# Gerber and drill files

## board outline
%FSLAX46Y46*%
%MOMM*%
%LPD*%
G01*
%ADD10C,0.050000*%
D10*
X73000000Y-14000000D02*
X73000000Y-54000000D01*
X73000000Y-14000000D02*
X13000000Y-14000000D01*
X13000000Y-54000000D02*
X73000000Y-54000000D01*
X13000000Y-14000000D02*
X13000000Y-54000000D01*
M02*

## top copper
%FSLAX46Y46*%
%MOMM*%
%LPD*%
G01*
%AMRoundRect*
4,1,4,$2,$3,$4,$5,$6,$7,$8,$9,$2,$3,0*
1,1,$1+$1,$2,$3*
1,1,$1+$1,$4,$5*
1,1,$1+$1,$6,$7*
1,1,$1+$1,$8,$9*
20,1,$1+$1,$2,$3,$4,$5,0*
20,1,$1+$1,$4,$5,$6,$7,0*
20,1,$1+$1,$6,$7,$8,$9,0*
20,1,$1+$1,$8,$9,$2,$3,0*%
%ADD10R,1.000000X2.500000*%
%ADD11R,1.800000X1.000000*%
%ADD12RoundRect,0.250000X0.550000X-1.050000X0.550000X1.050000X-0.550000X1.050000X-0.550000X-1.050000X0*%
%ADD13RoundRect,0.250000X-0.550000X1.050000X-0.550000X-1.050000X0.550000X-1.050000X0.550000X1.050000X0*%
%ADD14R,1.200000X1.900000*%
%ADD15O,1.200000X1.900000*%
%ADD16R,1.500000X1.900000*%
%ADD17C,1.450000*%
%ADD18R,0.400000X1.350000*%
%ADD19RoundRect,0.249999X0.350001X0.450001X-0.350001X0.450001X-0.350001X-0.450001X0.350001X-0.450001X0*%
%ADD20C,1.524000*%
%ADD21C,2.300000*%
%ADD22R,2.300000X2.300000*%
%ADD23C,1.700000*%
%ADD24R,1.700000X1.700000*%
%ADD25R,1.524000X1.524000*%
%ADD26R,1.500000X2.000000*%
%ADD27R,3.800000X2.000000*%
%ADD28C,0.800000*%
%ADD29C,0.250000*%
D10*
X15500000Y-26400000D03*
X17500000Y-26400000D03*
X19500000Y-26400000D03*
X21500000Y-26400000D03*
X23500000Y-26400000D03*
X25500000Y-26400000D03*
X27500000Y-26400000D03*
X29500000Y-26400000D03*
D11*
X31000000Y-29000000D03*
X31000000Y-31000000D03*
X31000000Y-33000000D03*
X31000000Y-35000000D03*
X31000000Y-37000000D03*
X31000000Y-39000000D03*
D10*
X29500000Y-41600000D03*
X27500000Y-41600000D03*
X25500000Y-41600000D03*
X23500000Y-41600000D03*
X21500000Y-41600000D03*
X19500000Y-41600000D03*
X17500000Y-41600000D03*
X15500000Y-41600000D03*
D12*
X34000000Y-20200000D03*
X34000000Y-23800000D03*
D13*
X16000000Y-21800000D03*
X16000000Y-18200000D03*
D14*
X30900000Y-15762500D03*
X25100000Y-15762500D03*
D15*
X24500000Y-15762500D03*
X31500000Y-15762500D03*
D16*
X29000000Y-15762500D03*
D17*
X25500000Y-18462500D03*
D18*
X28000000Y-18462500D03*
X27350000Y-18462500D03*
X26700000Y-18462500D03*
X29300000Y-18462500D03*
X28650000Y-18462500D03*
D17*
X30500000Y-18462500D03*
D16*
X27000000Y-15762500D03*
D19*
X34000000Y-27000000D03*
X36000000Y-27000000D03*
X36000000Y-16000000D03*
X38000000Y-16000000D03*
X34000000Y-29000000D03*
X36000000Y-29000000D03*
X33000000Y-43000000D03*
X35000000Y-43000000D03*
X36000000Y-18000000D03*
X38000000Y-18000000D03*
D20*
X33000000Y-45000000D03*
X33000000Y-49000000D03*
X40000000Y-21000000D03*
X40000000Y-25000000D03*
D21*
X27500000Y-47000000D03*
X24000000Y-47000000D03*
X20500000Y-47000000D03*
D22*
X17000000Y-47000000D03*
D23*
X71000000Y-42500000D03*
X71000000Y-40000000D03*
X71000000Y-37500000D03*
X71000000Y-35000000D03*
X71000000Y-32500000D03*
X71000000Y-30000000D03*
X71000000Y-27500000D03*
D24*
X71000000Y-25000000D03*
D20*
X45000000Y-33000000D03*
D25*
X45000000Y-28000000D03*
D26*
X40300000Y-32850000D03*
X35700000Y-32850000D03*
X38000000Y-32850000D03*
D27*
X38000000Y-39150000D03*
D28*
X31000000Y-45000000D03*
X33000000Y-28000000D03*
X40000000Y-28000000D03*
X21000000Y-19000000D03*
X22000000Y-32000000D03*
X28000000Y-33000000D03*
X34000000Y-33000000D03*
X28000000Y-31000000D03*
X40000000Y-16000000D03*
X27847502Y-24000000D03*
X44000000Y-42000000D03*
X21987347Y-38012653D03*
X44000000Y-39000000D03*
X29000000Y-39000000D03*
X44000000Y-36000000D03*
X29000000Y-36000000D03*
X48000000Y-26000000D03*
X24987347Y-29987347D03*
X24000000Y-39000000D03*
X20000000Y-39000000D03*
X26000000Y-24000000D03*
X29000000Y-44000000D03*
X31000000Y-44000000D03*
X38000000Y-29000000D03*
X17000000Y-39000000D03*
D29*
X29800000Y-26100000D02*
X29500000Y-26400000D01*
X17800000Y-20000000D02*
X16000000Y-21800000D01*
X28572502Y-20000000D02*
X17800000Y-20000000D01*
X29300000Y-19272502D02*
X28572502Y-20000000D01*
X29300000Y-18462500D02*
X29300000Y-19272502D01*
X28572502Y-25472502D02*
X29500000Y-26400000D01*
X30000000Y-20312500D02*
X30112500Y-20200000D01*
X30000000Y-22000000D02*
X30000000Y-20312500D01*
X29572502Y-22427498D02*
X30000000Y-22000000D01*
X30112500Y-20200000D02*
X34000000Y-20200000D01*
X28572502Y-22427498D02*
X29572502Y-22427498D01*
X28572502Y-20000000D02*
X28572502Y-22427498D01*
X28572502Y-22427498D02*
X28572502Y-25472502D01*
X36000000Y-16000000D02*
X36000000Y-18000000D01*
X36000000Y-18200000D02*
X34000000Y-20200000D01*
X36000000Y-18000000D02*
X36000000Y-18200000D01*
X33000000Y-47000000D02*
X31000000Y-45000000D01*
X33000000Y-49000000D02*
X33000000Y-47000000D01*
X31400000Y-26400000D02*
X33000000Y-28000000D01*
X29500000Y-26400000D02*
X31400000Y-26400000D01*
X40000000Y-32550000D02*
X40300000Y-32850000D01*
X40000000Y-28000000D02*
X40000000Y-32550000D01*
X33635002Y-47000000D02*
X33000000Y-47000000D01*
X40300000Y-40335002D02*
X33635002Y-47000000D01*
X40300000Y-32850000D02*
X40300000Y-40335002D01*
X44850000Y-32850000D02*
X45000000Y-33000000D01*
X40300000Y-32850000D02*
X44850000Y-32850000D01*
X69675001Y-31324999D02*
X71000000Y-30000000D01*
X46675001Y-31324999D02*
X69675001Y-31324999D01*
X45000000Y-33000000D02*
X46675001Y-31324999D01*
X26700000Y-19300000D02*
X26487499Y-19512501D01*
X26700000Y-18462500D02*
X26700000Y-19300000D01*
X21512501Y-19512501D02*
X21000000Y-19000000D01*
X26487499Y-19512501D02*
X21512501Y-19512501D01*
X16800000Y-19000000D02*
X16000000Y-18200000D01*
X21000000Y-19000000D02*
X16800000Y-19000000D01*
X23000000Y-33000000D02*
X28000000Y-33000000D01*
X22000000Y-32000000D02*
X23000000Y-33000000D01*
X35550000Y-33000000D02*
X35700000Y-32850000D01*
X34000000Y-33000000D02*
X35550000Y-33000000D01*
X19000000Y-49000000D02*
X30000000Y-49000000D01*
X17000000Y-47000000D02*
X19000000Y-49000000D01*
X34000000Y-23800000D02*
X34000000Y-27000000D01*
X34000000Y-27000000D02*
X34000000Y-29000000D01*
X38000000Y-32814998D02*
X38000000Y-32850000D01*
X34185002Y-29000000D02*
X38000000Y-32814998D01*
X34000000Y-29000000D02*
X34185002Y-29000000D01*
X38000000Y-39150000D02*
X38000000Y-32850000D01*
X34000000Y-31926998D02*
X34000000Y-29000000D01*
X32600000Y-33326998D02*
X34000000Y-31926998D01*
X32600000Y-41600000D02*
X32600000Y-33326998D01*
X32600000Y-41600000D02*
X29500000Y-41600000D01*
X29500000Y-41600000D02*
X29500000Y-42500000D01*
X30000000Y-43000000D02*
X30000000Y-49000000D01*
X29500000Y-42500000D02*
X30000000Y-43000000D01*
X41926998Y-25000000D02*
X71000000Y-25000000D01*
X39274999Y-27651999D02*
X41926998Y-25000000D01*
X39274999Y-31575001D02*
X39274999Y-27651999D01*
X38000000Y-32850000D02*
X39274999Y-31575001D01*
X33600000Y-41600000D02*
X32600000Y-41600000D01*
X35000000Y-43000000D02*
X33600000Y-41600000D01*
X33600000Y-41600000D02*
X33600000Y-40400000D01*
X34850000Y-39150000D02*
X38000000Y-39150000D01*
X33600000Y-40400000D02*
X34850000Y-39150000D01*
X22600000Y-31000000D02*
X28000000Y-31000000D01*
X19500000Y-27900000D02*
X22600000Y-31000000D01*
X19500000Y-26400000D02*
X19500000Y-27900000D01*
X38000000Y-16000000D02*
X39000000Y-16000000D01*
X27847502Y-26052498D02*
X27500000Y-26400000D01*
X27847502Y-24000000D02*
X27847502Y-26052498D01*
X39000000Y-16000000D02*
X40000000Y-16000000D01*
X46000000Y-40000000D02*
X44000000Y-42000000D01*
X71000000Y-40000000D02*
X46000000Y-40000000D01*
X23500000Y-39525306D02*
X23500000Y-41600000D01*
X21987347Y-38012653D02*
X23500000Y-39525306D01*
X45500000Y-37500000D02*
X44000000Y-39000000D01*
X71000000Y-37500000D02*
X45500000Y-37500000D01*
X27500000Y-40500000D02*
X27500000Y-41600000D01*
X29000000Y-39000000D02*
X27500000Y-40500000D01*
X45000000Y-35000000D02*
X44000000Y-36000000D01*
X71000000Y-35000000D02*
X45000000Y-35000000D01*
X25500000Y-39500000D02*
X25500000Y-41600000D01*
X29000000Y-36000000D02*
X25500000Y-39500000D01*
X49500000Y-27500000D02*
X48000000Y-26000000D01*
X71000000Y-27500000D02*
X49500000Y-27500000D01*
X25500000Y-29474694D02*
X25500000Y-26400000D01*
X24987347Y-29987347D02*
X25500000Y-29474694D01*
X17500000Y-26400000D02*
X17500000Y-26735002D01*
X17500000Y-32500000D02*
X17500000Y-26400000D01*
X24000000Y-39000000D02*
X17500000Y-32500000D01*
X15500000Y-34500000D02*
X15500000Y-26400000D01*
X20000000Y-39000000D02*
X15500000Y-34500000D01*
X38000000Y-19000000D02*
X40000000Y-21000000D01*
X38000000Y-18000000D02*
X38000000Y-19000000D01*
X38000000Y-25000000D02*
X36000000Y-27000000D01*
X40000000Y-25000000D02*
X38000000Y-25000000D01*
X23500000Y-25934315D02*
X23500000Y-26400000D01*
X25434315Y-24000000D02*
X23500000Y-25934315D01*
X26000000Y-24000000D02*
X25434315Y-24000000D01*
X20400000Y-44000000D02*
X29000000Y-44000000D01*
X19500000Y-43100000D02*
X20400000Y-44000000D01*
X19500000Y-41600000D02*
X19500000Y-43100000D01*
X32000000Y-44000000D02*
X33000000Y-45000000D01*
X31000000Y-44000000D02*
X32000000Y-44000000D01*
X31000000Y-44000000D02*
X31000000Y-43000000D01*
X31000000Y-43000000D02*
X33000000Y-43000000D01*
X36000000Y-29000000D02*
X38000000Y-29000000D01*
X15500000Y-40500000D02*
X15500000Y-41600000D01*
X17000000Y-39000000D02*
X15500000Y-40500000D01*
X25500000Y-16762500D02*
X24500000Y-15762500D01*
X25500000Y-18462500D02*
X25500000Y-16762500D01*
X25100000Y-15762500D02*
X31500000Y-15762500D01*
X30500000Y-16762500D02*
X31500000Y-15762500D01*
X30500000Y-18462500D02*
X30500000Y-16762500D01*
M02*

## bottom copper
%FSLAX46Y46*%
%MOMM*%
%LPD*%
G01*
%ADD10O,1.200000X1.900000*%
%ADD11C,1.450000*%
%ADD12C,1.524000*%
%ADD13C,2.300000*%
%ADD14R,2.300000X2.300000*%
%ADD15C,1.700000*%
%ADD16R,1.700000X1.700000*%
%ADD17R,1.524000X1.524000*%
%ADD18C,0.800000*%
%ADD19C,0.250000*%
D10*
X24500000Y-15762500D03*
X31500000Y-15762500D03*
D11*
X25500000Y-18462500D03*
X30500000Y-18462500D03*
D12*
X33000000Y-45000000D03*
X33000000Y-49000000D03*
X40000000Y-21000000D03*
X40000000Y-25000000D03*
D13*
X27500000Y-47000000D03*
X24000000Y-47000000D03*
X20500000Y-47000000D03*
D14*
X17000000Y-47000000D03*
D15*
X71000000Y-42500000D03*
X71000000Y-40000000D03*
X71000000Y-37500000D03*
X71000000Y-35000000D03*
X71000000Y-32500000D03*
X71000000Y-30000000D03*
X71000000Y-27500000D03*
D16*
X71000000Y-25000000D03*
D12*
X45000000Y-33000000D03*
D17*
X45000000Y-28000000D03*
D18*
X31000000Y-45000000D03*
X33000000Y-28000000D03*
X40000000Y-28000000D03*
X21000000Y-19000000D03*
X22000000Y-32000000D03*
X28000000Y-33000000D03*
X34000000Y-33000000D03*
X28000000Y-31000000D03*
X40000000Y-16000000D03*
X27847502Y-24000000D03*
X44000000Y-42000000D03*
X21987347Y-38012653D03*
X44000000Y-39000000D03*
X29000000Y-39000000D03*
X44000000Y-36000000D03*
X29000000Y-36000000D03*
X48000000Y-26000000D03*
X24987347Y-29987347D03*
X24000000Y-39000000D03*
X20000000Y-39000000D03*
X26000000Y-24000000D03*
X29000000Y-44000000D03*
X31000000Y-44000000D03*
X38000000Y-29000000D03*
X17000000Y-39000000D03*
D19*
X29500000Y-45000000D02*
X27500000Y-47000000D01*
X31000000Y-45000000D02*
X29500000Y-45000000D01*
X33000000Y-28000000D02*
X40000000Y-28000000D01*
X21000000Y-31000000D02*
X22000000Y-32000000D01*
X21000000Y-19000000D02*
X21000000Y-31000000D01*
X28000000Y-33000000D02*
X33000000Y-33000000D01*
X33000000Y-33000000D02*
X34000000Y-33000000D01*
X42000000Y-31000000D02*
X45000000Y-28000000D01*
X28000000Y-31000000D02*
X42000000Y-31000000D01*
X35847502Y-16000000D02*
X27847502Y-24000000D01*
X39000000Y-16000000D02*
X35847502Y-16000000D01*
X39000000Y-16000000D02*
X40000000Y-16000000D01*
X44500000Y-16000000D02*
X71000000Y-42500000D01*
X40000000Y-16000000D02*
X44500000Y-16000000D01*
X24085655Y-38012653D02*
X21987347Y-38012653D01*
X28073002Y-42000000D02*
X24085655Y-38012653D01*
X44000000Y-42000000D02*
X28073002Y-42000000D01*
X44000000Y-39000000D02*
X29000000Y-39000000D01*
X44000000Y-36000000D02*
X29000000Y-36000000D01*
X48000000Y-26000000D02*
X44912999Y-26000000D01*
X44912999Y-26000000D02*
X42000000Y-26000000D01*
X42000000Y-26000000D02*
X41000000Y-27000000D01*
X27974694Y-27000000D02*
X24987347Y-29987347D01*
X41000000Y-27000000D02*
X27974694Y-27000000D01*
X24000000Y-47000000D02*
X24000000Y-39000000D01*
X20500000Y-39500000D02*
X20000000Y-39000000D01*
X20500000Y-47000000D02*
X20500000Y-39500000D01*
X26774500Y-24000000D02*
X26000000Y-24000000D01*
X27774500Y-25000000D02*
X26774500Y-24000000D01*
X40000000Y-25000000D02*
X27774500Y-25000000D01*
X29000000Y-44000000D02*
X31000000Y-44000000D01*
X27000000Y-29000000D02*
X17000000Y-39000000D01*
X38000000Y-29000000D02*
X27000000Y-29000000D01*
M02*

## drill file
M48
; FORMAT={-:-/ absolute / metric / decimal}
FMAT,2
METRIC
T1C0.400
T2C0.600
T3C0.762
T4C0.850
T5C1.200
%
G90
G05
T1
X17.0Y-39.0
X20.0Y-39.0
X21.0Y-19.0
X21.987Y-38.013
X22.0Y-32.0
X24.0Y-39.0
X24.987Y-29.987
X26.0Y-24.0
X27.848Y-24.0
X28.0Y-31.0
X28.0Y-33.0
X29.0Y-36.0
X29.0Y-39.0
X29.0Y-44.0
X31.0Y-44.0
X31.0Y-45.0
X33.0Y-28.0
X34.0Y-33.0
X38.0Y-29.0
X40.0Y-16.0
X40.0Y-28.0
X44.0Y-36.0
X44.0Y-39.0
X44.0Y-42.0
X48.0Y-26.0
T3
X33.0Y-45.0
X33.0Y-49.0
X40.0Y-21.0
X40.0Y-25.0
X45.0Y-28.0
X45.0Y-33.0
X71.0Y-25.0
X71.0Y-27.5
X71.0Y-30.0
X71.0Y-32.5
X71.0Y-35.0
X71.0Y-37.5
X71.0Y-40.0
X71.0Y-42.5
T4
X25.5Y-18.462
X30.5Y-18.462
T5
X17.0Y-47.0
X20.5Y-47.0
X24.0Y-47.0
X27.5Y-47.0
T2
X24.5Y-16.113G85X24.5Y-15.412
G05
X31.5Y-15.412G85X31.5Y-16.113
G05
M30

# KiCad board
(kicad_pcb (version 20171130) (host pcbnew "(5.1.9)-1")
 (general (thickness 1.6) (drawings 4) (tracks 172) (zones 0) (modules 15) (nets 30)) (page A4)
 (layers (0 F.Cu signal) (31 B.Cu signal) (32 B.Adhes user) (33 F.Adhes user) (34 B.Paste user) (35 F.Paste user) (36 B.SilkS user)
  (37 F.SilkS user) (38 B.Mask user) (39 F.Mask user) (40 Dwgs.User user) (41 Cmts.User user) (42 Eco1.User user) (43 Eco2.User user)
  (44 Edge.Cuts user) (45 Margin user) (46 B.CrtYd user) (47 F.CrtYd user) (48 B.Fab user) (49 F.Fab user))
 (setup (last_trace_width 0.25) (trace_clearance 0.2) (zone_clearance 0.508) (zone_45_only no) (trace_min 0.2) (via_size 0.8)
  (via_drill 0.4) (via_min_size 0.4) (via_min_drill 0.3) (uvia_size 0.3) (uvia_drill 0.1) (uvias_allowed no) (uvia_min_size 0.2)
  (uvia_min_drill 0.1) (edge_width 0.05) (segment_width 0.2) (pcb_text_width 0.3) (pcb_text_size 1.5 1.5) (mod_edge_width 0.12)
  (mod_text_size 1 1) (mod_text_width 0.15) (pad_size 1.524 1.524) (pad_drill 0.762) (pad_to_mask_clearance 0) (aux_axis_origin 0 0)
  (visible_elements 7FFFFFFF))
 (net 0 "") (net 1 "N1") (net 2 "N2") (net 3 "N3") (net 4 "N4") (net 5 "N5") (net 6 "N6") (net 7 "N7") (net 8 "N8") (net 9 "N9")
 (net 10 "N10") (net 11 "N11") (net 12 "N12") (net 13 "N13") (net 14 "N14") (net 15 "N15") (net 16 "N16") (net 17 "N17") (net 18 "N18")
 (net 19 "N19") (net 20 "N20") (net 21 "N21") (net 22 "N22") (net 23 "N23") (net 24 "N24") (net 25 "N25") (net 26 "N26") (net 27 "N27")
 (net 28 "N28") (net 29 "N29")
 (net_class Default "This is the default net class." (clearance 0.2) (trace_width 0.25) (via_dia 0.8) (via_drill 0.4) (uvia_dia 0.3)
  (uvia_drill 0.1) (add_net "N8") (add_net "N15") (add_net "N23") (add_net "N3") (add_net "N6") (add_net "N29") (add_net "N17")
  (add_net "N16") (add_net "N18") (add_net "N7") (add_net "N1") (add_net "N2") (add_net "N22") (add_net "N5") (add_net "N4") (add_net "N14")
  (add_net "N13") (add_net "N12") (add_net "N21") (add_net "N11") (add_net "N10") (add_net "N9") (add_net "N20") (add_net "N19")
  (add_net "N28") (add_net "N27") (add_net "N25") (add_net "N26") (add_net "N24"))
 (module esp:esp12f (layer F.Cu) (at 19 34 90)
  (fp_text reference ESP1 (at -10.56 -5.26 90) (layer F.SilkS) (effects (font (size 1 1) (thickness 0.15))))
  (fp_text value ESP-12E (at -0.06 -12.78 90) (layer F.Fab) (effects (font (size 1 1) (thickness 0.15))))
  (pad 16 smd rect (at 7.6 -3.5 90) (size 2.5 1) (layers F.Cu F.Paste F.Mask) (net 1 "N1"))
  (pad 15 smd rect (at 7.6 -1.5 90) (size 2.5 1) (layers F.Cu F.Paste F.Mask) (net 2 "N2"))
  (pad 14 smd rect (at 7.6 0.5 90) (size 2.5 1) (layers F.Cu F.Paste F.Mask) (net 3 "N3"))
  (pad 13 smd rect (at 7.6 2.5 90) (size 2.5 1) (layers F.Cu F.Paste F.Mask) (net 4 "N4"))
  (pad 12 smd rect (at 7.6 4.5 90) (size 2.5 1) (layers F.Cu F.Paste F.Mask) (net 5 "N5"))
  (pad 11 smd rect (at 7.6 6.5 90) (size 2.5 1) (layers F.Cu F.Paste F.Mask) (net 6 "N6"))
  (pad 10 smd rect (at 7.6 8.5 90) (size 2.5 1) (layers F.Cu F.Paste F.Mask) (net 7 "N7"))
  (pad 9 smd rect (at 7.6 10.5 90) (size 2.5 1) (layers F.Cu F.Paste F.Mask) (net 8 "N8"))
  (pad 22 smd rect (at 5 12 90) (size 1 1.8) (layers F.Cu F.Paste F.Mask) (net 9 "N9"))
  (pad 21 smd rect (at 3 12 90) (size 1 1.8) (layers F.Cu F.Paste F.Mask) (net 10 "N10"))
  (pad 20 smd rect (at 1 12 90) (size 1 1.8) (layers F.Cu F.Paste F.Mask) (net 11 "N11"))
  (pad 19 smd rect (at -1 12 90) (size 1 1.8) (layers F.Cu F.Paste F.Mask) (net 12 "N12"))
  (pad 18 smd rect (at -3 12 90) (size 1 1.8) (layers F.Cu F.Paste F.Mask) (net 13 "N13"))
  (pad 17 smd rect (at -5 12 90) (size 1 1.8) (layers F.Cu F.Paste F.Mask) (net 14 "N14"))
  (pad 8 smd rect (at -7.6 10.5 90) (size 2.5 1) (layers F.Cu F.Paste F.Mask) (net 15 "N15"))
  (pad 7 smd rect (at -7.6 8.5 90) (size 2.5 1) (layers F.Cu F.Paste F.Mask) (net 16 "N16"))
  (pad 6 smd rect (at -7.6 6.5 90) (size 2.5 1) (layers F.Cu F.Paste F.Mask) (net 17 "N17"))
  (pad 5 smd rect (at -7.6 4.5 90) (size 2.5 1) (layers F.Cu F.Paste F.Mask) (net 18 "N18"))
  (pad 4 smd rect (at -7.6 2.5 90) (size 2.5 1) (layers F.Cu F.Paste F.Mask) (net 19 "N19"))
  (pad 3 smd rect (at -7.6 0.5 90) (size 2.5 1) (layers F.Cu F.Paste F.Mask) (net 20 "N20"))
  (pad 2 smd rect (at -7.6 -1.5 90) (size 2.5 1) (layers F.Cu F.Paste F.Mask) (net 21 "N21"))
  (pad 1 smd rect (at -7.6 -3.5 90) (size 2.5 1) (layers F.Cu F.Paste F.Mask) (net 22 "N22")))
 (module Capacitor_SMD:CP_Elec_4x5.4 (layer F.Cu) (at 34 22 90)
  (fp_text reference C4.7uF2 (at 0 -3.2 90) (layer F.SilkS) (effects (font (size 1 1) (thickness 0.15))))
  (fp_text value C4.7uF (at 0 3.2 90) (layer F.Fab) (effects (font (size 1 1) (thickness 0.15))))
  (pad 2 smd roundrect (at 1.8 0 90) (size 2.6 1.6) (layers F.Cu F.Paste F.Mask) (roundrect_rratio 0.15625) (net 8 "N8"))
  (pad 1 smd roundrect (at -1.8 0 90) (size 2.6 1.6) (layers F.Cu F.Paste F.Mask) (roundrect_rratio 0.15625) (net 15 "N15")))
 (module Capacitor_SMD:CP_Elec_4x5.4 (layer F.Cu) (at 16 20 270)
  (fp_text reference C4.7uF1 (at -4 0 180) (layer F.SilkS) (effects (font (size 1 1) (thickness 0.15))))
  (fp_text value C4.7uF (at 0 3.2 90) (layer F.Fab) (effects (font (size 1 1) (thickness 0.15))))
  (pad 2 smd roundrect (at 1.8 0 270) (size 2.6 1.6) (layers F.Cu F.Paste F.Mask) (roundrect_rratio 0.15625) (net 8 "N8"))
  (pad 1 smd roundrect (at -1.8 0 270) (size 2.6 1.6) (layers F.Cu F.Paste F.Mask) (roundrect_rratio 0.15625) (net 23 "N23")))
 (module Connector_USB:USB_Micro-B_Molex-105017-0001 (layer F.Cu) (at 28 17 180)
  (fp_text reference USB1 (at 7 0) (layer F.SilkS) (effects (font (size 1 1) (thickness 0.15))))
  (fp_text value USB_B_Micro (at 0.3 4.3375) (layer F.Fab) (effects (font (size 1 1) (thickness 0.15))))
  (pad 6 smd rect (at -2.9 1.2375 180) (size 1.2 1.9) (layers F.Cu F.Mask) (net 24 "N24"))
  (pad 6 smd rect (at 2.9 1.2375 180) (size 1.2 1.9) (layers F.Cu F.Mask) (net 24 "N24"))
  (pad 6 thru_hole oval (at 3.5 1.2375 180) (size 1.2 1.9) (drill oval 0.6 1.3) (layers *.Cu *.Mask) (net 24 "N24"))
  (pad 6 thru_hole oval (at -3.5 1.2375) (size 1.2 1.9) (drill oval 0.6 1.3) (layers *.Cu *.Mask) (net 24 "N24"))
  (pad 6 smd rect (at -1 1.2375 180) (size 1.5 1.9) (layers F.Cu F.Paste F.Mask) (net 24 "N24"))
  (pad 6 thru_hole circle (at 2.5 -1.4625 180) (size 1.45 1.45) (drill 0.85) (layers *.Cu *.Mask) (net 24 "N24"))
  (pad 3 smd rect (at 0 -1.4625 180) (size 0.4 1.35) (layers F.Cu F.Paste F.Mask) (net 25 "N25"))
  (pad 4 smd rect (at 0.65 -1.4625 180) (size 0.4 1.35) (layers F.Cu F.Paste F.Mask) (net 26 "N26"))
  (pad 5 smd rect (at 1.3 -1.4625 180) (size 0.4 1.35) (layers F.Cu F.Paste F.Mask) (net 23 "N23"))
  (pad 1 smd rect (at -1.3 -1.4625 180) (size 0.4 1.35) (layers F.Cu F.Paste F.Mask) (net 8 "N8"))
  (pad 2 smd rect (at -0.65 -1.4625 180) (size 0.4 1.35) (layers F.Cu F.Paste F.Mask) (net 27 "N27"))
  (pad 6 thru_hole circle (at -2.5 -1.4625 180) (size 1.45 1.45) (drill 0.85) (layers *.Cu *.Mask) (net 24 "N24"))
  (pad 6 smd rect (at 1 1.2375 180) (size 1.5 1.9) (layers F.Cu F.Paste F.Mask) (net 24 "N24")))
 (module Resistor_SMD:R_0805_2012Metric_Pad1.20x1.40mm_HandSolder (layer F.Cu) (at 35 27 180)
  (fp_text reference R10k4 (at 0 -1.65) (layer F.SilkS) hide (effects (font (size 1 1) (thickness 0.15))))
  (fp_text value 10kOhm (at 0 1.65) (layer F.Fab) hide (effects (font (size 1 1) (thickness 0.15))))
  (pad 2 smd roundrect (at 1 0 180) (size 1.2 1.4) (layers F.Cu F.Paste F.Mask) (roundrect_rratio 0.2083325) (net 15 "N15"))
  (pad 1 smd roundrect (at -1 0 180) (size 1.2 1.4) (layers F.Cu F.Paste F.Mask) (roundrect_rratio 0.2083325) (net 5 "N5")))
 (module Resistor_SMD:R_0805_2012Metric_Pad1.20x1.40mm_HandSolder (layer F.Cu) (at 37 16 180)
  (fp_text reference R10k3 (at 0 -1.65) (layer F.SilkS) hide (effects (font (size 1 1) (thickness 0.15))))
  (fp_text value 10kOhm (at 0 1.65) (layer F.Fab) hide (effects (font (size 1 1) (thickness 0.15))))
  (pad 2 smd roundrect (at 1 0 180) (size 1.2 1.4) (layers F.Cu F.Paste F.Mask) (roundrect_rratio 0.2083325) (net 8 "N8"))
  (pad 1 smd roundrect (at -1 0 180) (size 1.2 1.4) (layers F.Cu F.Paste F.Mask) (roundrect_rratio 0.2083325) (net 7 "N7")))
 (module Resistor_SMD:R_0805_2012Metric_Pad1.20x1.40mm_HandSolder (layer F.Cu) (at 35 29 180)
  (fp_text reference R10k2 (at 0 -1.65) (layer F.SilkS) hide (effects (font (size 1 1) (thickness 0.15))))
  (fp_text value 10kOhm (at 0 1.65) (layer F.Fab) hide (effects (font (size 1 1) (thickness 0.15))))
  (pad 2 smd roundrect (at 1 0 180) (size 1.2 1.4) (layers F.Cu F.Paste F.Mask) (roundrect_rratio 0.2083325) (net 15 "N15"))
  (pad 1 smd roundrect (at -1 0 180) (size 1.2 1.4) (layers F.Cu F.Paste F.Mask) (roundrect_rratio 0.2083325) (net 22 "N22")))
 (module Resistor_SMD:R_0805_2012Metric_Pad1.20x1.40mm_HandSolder (layer F.Cu) (at 34 43 180)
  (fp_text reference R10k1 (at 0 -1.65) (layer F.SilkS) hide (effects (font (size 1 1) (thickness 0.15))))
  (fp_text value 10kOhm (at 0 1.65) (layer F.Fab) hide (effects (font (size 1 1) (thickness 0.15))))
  (pad 2 smd roundrect (at 1 0 180) (size 1.2 1.4) (layers F.Cu F.Paste F.Mask) (roundrect_rratio 0.2083325) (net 20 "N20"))
  (pad 1 smd roundrect (at -1 0 180) (size 1.2 1.4) (layers F.Cu F.Paste F.Mask) (roundrect_rratio 0.2083325) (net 15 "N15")))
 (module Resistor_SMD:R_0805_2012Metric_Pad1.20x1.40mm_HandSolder (layer F.Cu) (at 37 18 180)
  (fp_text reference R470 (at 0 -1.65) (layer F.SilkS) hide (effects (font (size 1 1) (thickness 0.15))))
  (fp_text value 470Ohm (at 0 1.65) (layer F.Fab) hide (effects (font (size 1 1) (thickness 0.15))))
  (pad 2 smd roundrect (at 1 0 180) (size 1.2 1.4) (layers F.Cu F.Paste F.Mask) (roundrect_rratio 0.2083325) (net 8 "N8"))
  (pad 1 smd roundrect (at -1 0 180) (size 1.2 1.4) (layers F.Cu F.Paste F.Mask) (roundrect_rratio 0.2083325) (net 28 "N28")))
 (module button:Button (layer F.Cu) (at 33 47 180)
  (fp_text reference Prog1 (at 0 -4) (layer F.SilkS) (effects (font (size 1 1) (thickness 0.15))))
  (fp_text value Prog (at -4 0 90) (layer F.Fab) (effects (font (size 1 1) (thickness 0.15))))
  (pad 2 thru_hole circle (at 0 2 180) (size 1.524 1.524) (drill 0.762) (layers *.Cu *.Mask) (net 20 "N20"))
  (pad 1 thru_hole circle (at 0 -2 180) (size 1.524 1.524) (drill 0.762) (layers *.Cu *.Mask) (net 8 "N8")))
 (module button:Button (layer F.Cu) (at 40 23 180)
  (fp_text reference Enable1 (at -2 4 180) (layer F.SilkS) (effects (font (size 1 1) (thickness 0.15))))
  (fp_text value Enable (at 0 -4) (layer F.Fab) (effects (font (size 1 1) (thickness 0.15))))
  (pad 2 thru_hole circle (at 0 2 180) (size 1.524 1.524) (drill 0.762) (layers *.Cu *.Mask) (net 28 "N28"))
  (pad 1 thru_hole circle (at 0 -2 180) (size 1.524 1.524) (drill 0.762) (layers *.Cu *.Mask) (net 5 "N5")))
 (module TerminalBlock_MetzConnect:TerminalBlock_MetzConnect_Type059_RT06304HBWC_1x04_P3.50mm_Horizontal (layer F.Cu) (at 17 47)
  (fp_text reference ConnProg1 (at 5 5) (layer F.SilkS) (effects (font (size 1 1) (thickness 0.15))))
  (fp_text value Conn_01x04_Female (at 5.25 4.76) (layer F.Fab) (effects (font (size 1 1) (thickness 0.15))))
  (pad 4 thru_hole circle (at 10.5 0) (size 2.3 2.3) (drill 1.2) (layers *.Cu *.Mask) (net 8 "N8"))
  (pad 3 thru_hole circle (at 7 0) (size 2.3 2.3) (drill 1.2) (layers *.Cu *.Mask) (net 2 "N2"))
  (pad 2 thru_hole circle (at 3.5 0) (size 2.3 2.3) (drill 1.2) (layers *.Cu *.Mask) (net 1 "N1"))
  (pad 1 thru_hole rect (at 0 0) (size 2.3 2.3) (drill 1.2) (layers *.Cu *.Mask) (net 15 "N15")))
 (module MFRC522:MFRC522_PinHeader (layer F.Cu) (at 73 24 270)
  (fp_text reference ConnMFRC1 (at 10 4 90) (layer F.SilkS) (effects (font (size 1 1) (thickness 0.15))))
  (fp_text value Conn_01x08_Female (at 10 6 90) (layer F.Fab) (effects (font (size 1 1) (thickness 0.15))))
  (pad 8 thru_hole circle (at 18.5 2 270) (size 1.7 1.7) (drill 0.762) (layers *.Cu *.Mask) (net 7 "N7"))
  (pad 7 thru_hole circle (at 16 2 270) (size 1.7 1.7) (drill 0.762) (layers *.Cu *.Mask) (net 18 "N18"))
  (pad 6 thru_hole circle (at 13.5 2 270) (size 1.7 1.7) (drill 0.762) (layers *.Cu *.Mask) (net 16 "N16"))
  (pad 5 thru_hole circle (at 11 2 270) (size 1.7 1.7) (drill 0.762) (layers *.Cu *.Mask) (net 17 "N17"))
  (pad 4 thru_hole circle (at 8.5 2 270) (size 1.7 1.7) (drill 0.762) (layers *.Cu *.Mask) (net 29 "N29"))
  (pad 3 thru_hole circle (at 6 2 270) (size 1.7 1.7) (drill 0.762) (layers *.Cu *.Mask) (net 8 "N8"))
  (pad 2 thru_hole circle (at 3.5 2 270) (size 1.7 1.7) (drill 0.762) (layers *.Cu *.Mask) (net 6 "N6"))
  (pad 1 thru_hole rect (at 1 2 270) (size 1.7 1.7) (drill 0.762) (layers *.Cu *.Mask) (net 15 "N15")))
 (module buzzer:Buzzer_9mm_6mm (layer F.Cu) (at 46 27 270)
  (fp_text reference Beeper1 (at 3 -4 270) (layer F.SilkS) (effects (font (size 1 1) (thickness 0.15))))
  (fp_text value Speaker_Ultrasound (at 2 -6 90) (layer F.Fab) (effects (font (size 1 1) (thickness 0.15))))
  (pad 2 thru_hole circle (at 6 1 270) (size 1.524 1.524) (drill 0.762) (layers *.Cu *.Mask) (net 8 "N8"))
  (pad 1 thru_hole rect (at 1 1 270) (size 1.524 1.524) (drill 0.762) (layers *.Cu *.Mask) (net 3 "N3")))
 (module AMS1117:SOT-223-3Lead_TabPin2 (layer F.Cu) (at 38 36 270)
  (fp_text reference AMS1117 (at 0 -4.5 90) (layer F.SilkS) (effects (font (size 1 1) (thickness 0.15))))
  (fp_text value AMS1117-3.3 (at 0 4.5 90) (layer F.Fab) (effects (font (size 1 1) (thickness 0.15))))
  (pad 1 smd rect (at -3.15 -2.3 270) (size 2 1.5) (layers F.Cu F.Paste F.Mask) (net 8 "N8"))
  (pad 3 smd rect (at -3.15 2.3 270) (size 2 1.5) (layers F.Cu F.Paste F.Mask) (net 23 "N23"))
  (pad 2 smd rect (at -3.15 0 270) (size 2 1.5) (layers F.Cu F.Paste F.Mask) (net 15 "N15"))
  (pad 2 smd rect (at 3.15 0 270) (size 2 3.8) (layers F.Cu F.Paste F.Mask) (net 15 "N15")))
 (gr_line (start 73 14) (end 73 54) (layer Edge.Cuts) (width 0.05))
 (gr_line (start 73 14) (end 13 14) (layer Edge.Cuts) (width 0.05))
 (gr_line (start 13 54) (end 73 54) (layer Edge.Cuts) (width 0.05))
 (gr_line (start 13 14) (end 13 54) (layer Edge.Cuts) (width 0.05))
 (segment (start 29.8 26.1) (end 29.5 26.4) (width 0.25) (layer F.Cu) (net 8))
 (segment (start 17.8 20) (end 16 21.8) (width 0.25) (layer F.Cu) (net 8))
 (segment (start 28.572502 20) (end 17.8 20) (width 0.25) (layer F.Cu) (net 8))
 (segment (start 29.3 19.272502) (end 28.572502 20) (width 0.25) (layer F.Cu) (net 8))
 (segment (start 29.3 18.4625) (end 29.3 19.272502) (width 0.25) (layer F.Cu) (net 8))
 (segment (start 28.572502 25.472502) (end 29.5 26.4) (width 0.25) (layer F.Cu) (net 8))
 (segment (start 30 20.3125) (end 30.1125 20.2) (width 0.25) (layer F.Cu) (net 8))
 (segment (start 30 22) (end 30 20.3125) (width 0.25) (layer F.Cu) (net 8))
 (segment (start 29.572502 22.427498) (end 30 22) (width 0.25) (layer F.Cu) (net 8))
 (segment (start 30.1125 20.2) (end 34 20.2) (width 0.25) (layer F.Cu) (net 8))
 (segment (start 28.572502 22.427498) (end 29.572502 22.427498) (width 0.25) (layer F.Cu) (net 8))
 (segment (start 28.572502 20) (end 28.572502 22.427498) (width 0.25) (layer F.Cu) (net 8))
 (segment (start 28.572502 22.427498) (end 28.572502 25.472502) (width 0.25) (layer F.Cu) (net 8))
 (segment (start 36 16) (end 36 18) (width 0.25) (layer F.Cu) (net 8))
 (segment (start 36 18.2) (end 34 20.2) (width 0.25) (layer F.Cu) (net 8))
 (segment (start 36 18) (end 36 18.2) (width 0.25) (layer F.Cu) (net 8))
 (via (at 31 45) (size 0.8) (drill 0.4) (layers F.Cu B.Cu) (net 8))
 (segment (start 33 47) (end 31 45) (width 0.25) (layer F.Cu) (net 8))
 (segment (start 33 49) (end 33 47) (width 0.25) (layer F.Cu) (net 8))
 (segment (start 29.5 45) (end 27.5 47) (width 0.25) (layer B.Cu) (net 8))
 (segment (start 31 45) (end 29.5 45) (width 0.25) (layer B.Cu) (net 8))
 (via (at 33 28) (size 0.8) (drill 0.4) (layers F.Cu B.Cu) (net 8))
 (segment (start 31.4 26.4) (end 33 28) (width 0.25) (layer F.Cu) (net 8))
 (segment (start 29.5 26.4) (end 31.4 26.4) (width 0.25) (layer F.Cu) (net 8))
 (via (at 40 28) (size 0.8) (drill 0.4) (layers F.Cu B.Cu) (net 8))
 (segment (start 33 28) (end 40 28) (width 0.25) (layer B.Cu) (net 8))
 (segment (start 40 32.55) (end 40.3 32.85) (width 0.25) (layer F.Cu) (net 8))
 (segment (start 40 28) (end 40 32.55) (width 0.25) (layer F.Cu) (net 8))
 (segment (start 33.635002 47) (end 33 47) (width 0.25) (layer F.Cu) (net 8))
 (segment (start 40.3 40.335002) (end 33.635002 47) (width 0.25) (layer F.Cu) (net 8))
 (segment (start 40.3 32.85) (end 40.3 40.335002) (width 0.25) (layer F.Cu) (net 8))
 (segment (start 44.85 32.85) (end 45 33) (width 0.25) (layer F.Cu) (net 8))
 (segment (start 40.3 32.85) (end 44.85 32.85) (width 0.25) (layer F.Cu) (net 8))
 (segment (start 69.675001 31.324999) (end 71 30) (width 0.25) (layer F.Cu) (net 8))
 (segment (start 46.675001 31.324999) (end 69.675001 31.324999) (width 0.25) (layer F.Cu) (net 8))
 (segment (start 45 33) (end 46.675001 31.324999) (width 0.25) (layer F.Cu) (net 8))
 (segment (start 26.7 19.3) (end 26.487499 19.512501) (width 0.25) (layer F.Cu) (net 23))
 (segment (start 26.7 18.4625) (end 26.7 19.3) (width 0.25) (layer F.Cu) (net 23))
 (via (at 21 19) (size 0.8) (drill 0.4) (layers F.Cu B.Cu) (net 23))
 (segment (start 21.512501 19.512501) (end 21 19) (width 0.25) (layer F.Cu) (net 23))
 (segment (start 26.487499 19.512501) (end 21.512501 19.512501) (width 0.25) (layer F.Cu) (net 23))
 (segment (start 16.8 19) (end 16 18.2) (width 0.25) (layer F.Cu) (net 23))
 (segment (start 21 19) (end 16.8 19) (width 0.25) (layer F.Cu) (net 23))
 (via (at 22 32) (size 0.8) (drill 0.4) (layers F.Cu B.Cu) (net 23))
 (segment (start 21 31) (end 22 32) (width 0.25) (layer B.Cu) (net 23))
 (segment (start 21 19) (end 21 31) (width 0.25) (layer B.Cu) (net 23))
 (via (at 28 33) (size 0.8) (drill 0.4) (layers F.Cu B.Cu) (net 23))
 (segment (start 23 33) (end 28 33) (width 0.25) (layer F.Cu) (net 23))
 (segment (start 22 32) (end 23 33) (width 0.25) (layer F.Cu) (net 23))
 (segment (start 28 33) (end 33 33) (width 0.25) (layer B.Cu) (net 23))
 (via (at 34 33) (size 0.8) (drill 0.4) (layers F.Cu B.Cu) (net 23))
 (segment (start 33 33) (end 34 33) (width 0.25) (layer B.Cu) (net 23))
 (segment (start 35.55 33) (end 35.7 32.85) (width 0.25) (layer F.Cu) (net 23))
 (segment (start 34 33) (end 35.55 33) (width 0.25) (layer F.Cu) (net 23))
 (segment (start 19 49) (end 30 49) (width 0.25) (layer F.Cu) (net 15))
 (segment (start 17 47) (end 19 49) (width 0.25) (layer F.Cu) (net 15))
 (segment (start 34 23.8) (end 34 27) (width 0.25) (layer F.Cu) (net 15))
 (segment (start 34 27) (end 34 29) (width 0.25) (layer F.Cu) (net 15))
 (segment (start 38 32.814998) (end 38 32.85) (width 0.25) (layer F.Cu) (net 15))
 (segment (start 34.185002 29) (end 38 32.814998) (width 0.25) (layer F.Cu) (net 15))
 (segment (start 34 29) (end 34.185002 29) (width 0.25) (layer F.Cu) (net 15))
 (segment (start 38 39.15) (end 38 32.85) (width 0.25) (layer F.Cu) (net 15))
 (segment (start 34 31.926998) (end 34 29) (width 0.25) (layer F.Cu) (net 15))
 (segment (start 32.6 33.326998) (end 34 31.926998) (width 0.25) (layer F.Cu) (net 15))
 (segment (start 32.6 41.6) (end 32.6 33.326998) (width 0.25) (layer F.Cu) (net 15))
 (segment (start 32.6 41.6) (end 29.5 41.6) (width 0.25) (layer F.Cu) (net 15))
 (segment (start 29.5 41.6) (end 29.5 42.5) (width 0.25) (layer F.Cu) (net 15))
 (segment (start 30 43) (end 30 49) (width 0.25) (layer F.Cu) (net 15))
 (segment (start 29.5 42.5) (end 30 43) (width 0.25) (layer F.Cu) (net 15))
 (segment (start 41.926998 25) (end 71 25) (width 0.25) (layer F.Cu) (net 15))
 (segment (start 39.274999 27.651999) (end 41.926998 25) (width 0.25) (layer F.Cu) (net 15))
 (segment (start 39.274999 31.575001) (end 39.274999 27.651999) (width 0.25) (layer F.Cu) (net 15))
 (segment (start 38 32.85) (end 39.274999 31.575001) (width 0.25) (layer F.Cu) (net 15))
 (segment (start 33.6 41.6) (end 32.6 41.6) (width 0.25) (layer F.Cu) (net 15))
 (segment (start 35 43) (end 33.6 41.6) (width 0.25) (layer F.Cu) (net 15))
 (segment (start 33.6 41.6) (end 33.6 40.4) (width 0.25) (layer F.Cu) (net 15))
 (segment (start 34.85 39.15) (end 38 39.15) (width 0.25) (layer F.Cu) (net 15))
 (segment (start 33.6 40.4) (end 34.85 39.15) (width 0.25) (layer F.Cu) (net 15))
 (segment (start 22.6 31) (end 28 31) (width 0.25) (layer F.Cu) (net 3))
 (via (at 28 31) (size 0.8) (drill 0.4) (layers F.Cu B.Cu) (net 3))
 (segment (start 19.5 27.9) (end 22.6 31) (width 0.25) (layer F.Cu) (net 3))
 (segment (start 19.5 26.4) (end 19.5 27.9) (width 0.25) (layer F.Cu) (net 3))
 (segment (start 42 31) (end 45 28) (width 0.25) (layer B.Cu) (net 3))
 (segment (start 28 31) (end 42 31) (width 0.25) (layer B.Cu) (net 3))
 (via (at 40 16) (size 0.8) (drill 0.4) (layers F.Cu B.Cu) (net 7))
 (segment (start 38 16) (end 39 16) (width 0.25) (layer F.Cu) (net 7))
 (via (at 27.847502 24) (size 0.8) (drill 0.4) (layers F.Cu B.Cu) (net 7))
 (segment (start 35.847502 16) (end 27.847502 24) (width 0.25) (layer B.Cu) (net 7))
 (segment (start 39 16) (end 35.847502 16) (width 0.25) (layer B.Cu) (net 7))
 (segment (start 27.847502 26.052498) (end 27.5 26.4) (width 0.25) (layer F.Cu) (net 7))
 (segment (start 27.847502 24) (end 27.847502 26.052498) (width 0.25) (layer F.Cu) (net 7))
 (segment (start 39 16) (end 40 16) (width 0.25) (layer F.Cu) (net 7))
 (segment (start 39 16) (end 40 16) (width 0.25) (layer B.Cu) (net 7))
 (segment (start 44.5 16) (end 71 42.5) (width 0.25) (layer B.Cu) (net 7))
 (segment (start 40 16) (end 44.5 16) (width 0.25) (layer B.Cu) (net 7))
 (via (at 44 42) (size 0.8) (drill 0.4) (layers F.Cu B.Cu) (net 18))
 (segment (start 46 40) (end 44 42) (width 0.25) (layer F.Cu) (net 18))
 (segment (start 71 40) (end 46 40) (width 0.25) (layer F.Cu) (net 18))
 (via (at 21.987347 38.012653) (size 0.8) (drill 0.4) (layers F.Cu B.Cu) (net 18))
 (segment (start 24.085655 38.012653) (end 21.987347 38.012653) (width 0.25) (layer B.Cu) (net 18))
 (segment (start 28.073002 42) (end 24.085655 38.012653) (width 0.25) (layer B.Cu) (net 18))
 (segment (start 44 42) (end 28.073002 42) (width 0.25) (layer B.Cu) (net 18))
 (segment (start 23.5 39.525306) (end 23.5 41.6) (width 0.25) (layer F.Cu) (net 18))
 (segment (start 21.987347 38.012653) (end 23.5 39.525306) (width 0.25) (layer F.Cu) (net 18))
 (via (at 44 39) (size 0.8) (drill 0.4) (layers F.Cu B.Cu) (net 16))
 (segment (start 45.5 37.5) (end 44 39) (width 0.25) (layer F.Cu) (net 16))
 (segment (start 71 37.5) (end 45.5 37.5) (width 0.25) (layer F.Cu) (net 16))
 (via (at 29 39) (size 0.8) (drill 0.4) (layers F.Cu B.Cu) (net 16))
 (segment (start 44 39) (end 29 39) (width 0.25) (layer B.Cu) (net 16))
 (segment (start 27.5 40.5) (end 27.5 41.6) (width 0.25) (layer F.Cu) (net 16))
 (segment (start 29 39) (end 27.5 40.5) (width 0.25) (layer F.Cu) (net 16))
 (via (at 44 36) (size 0.8) (drill 0.4) (layers F.Cu B.Cu) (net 17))
 (segment (start 45 35) (end 44 36) (width 0.25) (layer F.Cu) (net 17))
 (segment (start 71 35) (end 45 35) (width 0.25) (layer F.Cu) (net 17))
 (via (at 29 36) (size 0.8) (drill 0.4) (layers F.Cu B.Cu) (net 17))
 (segment (start 44 36) (end 29 36) (width 0.25) (layer B.Cu) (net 17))
 (segment (start 25.5 39.5) (end 25.5 41.6) (width 0.25) (layer F.Cu) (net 17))
 (segment (start 29 36) (end 25.5 39.5) (width 0.25) (layer F.Cu) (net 17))
 (via (at 48 26) (size 0.8) (drill 0.4) (layers F.Cu B.Cu) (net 6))
 (segment (start 49.5 27.5) (end 48 26) (width 0.25) (layer F.Cu) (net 6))
 (segment (start 71 27.5) (end 49.5 27.5) (width 0.25) (layer F.Cu) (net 6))
 (segment (start 48 26) (end 44.912999 26) (width 0.25) (layer B.Cu) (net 6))
 (segment (start 44.912999 26) (end 42 26) (width 0.25) (layer B.Cu) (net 6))
 (segment (start 42 26) (end 41 27) (width 0.25) (layer B.Cu) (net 6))
 (via (at 24.987347 29.987347) (size 0.8) (drill 0.4) (layers F.Cu B.Cu) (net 6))
 (segment (start 27.974694 27) (end 24.987347 29.987347) (width 0.25) (layer B.Cu) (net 6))
 (segment (start 41 27) (end 27.974694 27) (width 0.25) (layer B.Cu) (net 6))
 (segment (start 25.5 29.474694) (end 25.5 26.4) (width 0.25) (layer F.Cu) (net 6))
 (segment (start 24.987347 29.987347) (end 25.5 29.474694) (width 0.25) (layer F.Cu) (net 6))
 (segment (start 17.5 26.4) (end 17.5 26.735002) (width 0.25) (layer F.Cu) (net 2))
 (via (at 24 39) (size 0.8) (drill 0.4) (layers F.Cu B.Cu) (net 2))
 (segment (start 24 47) (end 24 39) (width 0.25) (layer B.Cu) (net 2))
 (segment (start 17.5 32.5) (end 17.5 26.4) (width 0.25) (layer F.Cu) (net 2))
 (segment (start 24 39) (end 17.5 32.5) (width 0.25) (layer F.Cu) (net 2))
 (segment (start 20.5 39.5) (end 20 39) (width 0.25) (layer B.Cu) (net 1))
 (via (at 20 39) (size 0.8) (drill 0.4) (layers F.Cu B.Cu) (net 1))
 (segment (start 20.5 47) (end 20.5 39.5) (width 0.25) (layer B.Cu) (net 1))
 (segment (start 15.5 34.5) (end 15.5 26.4) (width 0.25) (layer F.Cu) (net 1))
 (segment (start 20 39) (end 15.5 34.5) (width 0.25) (layer F.Cu) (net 1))
 (segment (start 38 19) (end 40 21) (width 0.25) (layer F.Cu) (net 28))
 (segment (start 38 18) (end 38 19) (width 0.25) (layer F.Cu) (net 28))
 (segment (start 38 25) (end 36 27) (width 0.25) (layer F.Cu) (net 5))
 (segment (start 40 25) (end 38 25) (width 0.25) (layer F.Cu) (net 5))
 (via (at 26 24) (size 0.8) (drill 0.4) (layers F.Cu B.Cu) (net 5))
 (segment (start 26.7745 24) (end 26 24) (width 0.25) (layer B.Cu) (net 5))
 (segment (start 27.7745 25) (end 26.7745 24) (width 0.25) (layer B.Cu) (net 5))
 (segment (start 40 25) (end 27.7745 25) (width 0.25) (layer B.Cu) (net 5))
 (segment (start 23.5 25.934315) (end 23.5 26.4) (width 0.25) (layer F.Cu) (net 5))
 (segment (start 25.434315 24) (end 23.5 25.934315) (width 0.25) (layer F.Cu) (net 5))
 (segment (start 26 24) (end 25.434315 24) (width 0.25) (layer F.Cu) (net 5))
 (segment (start 20.4 44) (end 29 44) (width 0.25) (layer F.Cu) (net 20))
 (segment (start 19.5 43.1) (end 20.4 44) (width 0.25) (layer F.Cu) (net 20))
 (via (at 29 44) (size 0.8) (drill 0.4) (layers F.Cu B.Cu) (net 20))
 (segment (start 19.5 41.6) (end 19.5 43.1) (width 0.25) (layer F.Cu) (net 20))
 (via (at 31 44) (size 0.8) (drill 0.4) (layers F.Cu B.Cu) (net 20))
 (segment (start 29 44) (end 31 44) (width 0.25) (layer B.Cu) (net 20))
 (segment (start 32 44) (end 33 45) (width 0.25) (layer F.Cu) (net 20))
 (segment (start 31 44) (end 32 44) (width 0.25) (layer F.Cu) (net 20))
 (segment (start 31 44) (end 31 43) (width 0.25) (layer F.Cu) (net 20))
 (segment (start 31 43) (end 33 43) (width 0.25) (layer F.Cu) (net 20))
 (via (at 38 29) (size 0.8) (drill 0.4) (layers F.Cu B.Cu) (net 22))
 (segment (start 36 29) (end 38 29) (width 0.25) (layer F.Cu) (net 22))
 (via (at 17 39) (size 0.8) (drill 0.4) (layers F.Cu B.Cu) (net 22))
 (segment (start 27 29) (end 17 39) (width 0.25) (layer B.Cu) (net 22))
 (segment (start 38 29) (end 27 29) (width 0.25) (layer B.Cu) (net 22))
 (segment (start 15.5 40.5) (end 15.5 41.6) (width 0.25) (layer F.Cu) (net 22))
 (segment (start 17 39) (end 15.5 40.5) (width 0.25) (layer F.Cu) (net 22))
 (segment (start 25.5 16.7625) (end 24.5 15.7625) (width 0.25) (layer F.Cu) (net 24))
 (segment (start 25.5 18.4625) (end 25.5 16.7625) (width 0.25) (layer F.Cu) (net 24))
 (segment (start 25.1 15.7625) (end 31.5 15.7625) (width 0.25) (layer F.Cu) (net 24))
 (segment (start 30.5 16.7625) (end 31.5 15.7625) (width 0.25) (layer F.Cu) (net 24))
 (segment (start 30.5 18.4625) (end 30.5 16.7625) (width 0.25) (layer F.Cu) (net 24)))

